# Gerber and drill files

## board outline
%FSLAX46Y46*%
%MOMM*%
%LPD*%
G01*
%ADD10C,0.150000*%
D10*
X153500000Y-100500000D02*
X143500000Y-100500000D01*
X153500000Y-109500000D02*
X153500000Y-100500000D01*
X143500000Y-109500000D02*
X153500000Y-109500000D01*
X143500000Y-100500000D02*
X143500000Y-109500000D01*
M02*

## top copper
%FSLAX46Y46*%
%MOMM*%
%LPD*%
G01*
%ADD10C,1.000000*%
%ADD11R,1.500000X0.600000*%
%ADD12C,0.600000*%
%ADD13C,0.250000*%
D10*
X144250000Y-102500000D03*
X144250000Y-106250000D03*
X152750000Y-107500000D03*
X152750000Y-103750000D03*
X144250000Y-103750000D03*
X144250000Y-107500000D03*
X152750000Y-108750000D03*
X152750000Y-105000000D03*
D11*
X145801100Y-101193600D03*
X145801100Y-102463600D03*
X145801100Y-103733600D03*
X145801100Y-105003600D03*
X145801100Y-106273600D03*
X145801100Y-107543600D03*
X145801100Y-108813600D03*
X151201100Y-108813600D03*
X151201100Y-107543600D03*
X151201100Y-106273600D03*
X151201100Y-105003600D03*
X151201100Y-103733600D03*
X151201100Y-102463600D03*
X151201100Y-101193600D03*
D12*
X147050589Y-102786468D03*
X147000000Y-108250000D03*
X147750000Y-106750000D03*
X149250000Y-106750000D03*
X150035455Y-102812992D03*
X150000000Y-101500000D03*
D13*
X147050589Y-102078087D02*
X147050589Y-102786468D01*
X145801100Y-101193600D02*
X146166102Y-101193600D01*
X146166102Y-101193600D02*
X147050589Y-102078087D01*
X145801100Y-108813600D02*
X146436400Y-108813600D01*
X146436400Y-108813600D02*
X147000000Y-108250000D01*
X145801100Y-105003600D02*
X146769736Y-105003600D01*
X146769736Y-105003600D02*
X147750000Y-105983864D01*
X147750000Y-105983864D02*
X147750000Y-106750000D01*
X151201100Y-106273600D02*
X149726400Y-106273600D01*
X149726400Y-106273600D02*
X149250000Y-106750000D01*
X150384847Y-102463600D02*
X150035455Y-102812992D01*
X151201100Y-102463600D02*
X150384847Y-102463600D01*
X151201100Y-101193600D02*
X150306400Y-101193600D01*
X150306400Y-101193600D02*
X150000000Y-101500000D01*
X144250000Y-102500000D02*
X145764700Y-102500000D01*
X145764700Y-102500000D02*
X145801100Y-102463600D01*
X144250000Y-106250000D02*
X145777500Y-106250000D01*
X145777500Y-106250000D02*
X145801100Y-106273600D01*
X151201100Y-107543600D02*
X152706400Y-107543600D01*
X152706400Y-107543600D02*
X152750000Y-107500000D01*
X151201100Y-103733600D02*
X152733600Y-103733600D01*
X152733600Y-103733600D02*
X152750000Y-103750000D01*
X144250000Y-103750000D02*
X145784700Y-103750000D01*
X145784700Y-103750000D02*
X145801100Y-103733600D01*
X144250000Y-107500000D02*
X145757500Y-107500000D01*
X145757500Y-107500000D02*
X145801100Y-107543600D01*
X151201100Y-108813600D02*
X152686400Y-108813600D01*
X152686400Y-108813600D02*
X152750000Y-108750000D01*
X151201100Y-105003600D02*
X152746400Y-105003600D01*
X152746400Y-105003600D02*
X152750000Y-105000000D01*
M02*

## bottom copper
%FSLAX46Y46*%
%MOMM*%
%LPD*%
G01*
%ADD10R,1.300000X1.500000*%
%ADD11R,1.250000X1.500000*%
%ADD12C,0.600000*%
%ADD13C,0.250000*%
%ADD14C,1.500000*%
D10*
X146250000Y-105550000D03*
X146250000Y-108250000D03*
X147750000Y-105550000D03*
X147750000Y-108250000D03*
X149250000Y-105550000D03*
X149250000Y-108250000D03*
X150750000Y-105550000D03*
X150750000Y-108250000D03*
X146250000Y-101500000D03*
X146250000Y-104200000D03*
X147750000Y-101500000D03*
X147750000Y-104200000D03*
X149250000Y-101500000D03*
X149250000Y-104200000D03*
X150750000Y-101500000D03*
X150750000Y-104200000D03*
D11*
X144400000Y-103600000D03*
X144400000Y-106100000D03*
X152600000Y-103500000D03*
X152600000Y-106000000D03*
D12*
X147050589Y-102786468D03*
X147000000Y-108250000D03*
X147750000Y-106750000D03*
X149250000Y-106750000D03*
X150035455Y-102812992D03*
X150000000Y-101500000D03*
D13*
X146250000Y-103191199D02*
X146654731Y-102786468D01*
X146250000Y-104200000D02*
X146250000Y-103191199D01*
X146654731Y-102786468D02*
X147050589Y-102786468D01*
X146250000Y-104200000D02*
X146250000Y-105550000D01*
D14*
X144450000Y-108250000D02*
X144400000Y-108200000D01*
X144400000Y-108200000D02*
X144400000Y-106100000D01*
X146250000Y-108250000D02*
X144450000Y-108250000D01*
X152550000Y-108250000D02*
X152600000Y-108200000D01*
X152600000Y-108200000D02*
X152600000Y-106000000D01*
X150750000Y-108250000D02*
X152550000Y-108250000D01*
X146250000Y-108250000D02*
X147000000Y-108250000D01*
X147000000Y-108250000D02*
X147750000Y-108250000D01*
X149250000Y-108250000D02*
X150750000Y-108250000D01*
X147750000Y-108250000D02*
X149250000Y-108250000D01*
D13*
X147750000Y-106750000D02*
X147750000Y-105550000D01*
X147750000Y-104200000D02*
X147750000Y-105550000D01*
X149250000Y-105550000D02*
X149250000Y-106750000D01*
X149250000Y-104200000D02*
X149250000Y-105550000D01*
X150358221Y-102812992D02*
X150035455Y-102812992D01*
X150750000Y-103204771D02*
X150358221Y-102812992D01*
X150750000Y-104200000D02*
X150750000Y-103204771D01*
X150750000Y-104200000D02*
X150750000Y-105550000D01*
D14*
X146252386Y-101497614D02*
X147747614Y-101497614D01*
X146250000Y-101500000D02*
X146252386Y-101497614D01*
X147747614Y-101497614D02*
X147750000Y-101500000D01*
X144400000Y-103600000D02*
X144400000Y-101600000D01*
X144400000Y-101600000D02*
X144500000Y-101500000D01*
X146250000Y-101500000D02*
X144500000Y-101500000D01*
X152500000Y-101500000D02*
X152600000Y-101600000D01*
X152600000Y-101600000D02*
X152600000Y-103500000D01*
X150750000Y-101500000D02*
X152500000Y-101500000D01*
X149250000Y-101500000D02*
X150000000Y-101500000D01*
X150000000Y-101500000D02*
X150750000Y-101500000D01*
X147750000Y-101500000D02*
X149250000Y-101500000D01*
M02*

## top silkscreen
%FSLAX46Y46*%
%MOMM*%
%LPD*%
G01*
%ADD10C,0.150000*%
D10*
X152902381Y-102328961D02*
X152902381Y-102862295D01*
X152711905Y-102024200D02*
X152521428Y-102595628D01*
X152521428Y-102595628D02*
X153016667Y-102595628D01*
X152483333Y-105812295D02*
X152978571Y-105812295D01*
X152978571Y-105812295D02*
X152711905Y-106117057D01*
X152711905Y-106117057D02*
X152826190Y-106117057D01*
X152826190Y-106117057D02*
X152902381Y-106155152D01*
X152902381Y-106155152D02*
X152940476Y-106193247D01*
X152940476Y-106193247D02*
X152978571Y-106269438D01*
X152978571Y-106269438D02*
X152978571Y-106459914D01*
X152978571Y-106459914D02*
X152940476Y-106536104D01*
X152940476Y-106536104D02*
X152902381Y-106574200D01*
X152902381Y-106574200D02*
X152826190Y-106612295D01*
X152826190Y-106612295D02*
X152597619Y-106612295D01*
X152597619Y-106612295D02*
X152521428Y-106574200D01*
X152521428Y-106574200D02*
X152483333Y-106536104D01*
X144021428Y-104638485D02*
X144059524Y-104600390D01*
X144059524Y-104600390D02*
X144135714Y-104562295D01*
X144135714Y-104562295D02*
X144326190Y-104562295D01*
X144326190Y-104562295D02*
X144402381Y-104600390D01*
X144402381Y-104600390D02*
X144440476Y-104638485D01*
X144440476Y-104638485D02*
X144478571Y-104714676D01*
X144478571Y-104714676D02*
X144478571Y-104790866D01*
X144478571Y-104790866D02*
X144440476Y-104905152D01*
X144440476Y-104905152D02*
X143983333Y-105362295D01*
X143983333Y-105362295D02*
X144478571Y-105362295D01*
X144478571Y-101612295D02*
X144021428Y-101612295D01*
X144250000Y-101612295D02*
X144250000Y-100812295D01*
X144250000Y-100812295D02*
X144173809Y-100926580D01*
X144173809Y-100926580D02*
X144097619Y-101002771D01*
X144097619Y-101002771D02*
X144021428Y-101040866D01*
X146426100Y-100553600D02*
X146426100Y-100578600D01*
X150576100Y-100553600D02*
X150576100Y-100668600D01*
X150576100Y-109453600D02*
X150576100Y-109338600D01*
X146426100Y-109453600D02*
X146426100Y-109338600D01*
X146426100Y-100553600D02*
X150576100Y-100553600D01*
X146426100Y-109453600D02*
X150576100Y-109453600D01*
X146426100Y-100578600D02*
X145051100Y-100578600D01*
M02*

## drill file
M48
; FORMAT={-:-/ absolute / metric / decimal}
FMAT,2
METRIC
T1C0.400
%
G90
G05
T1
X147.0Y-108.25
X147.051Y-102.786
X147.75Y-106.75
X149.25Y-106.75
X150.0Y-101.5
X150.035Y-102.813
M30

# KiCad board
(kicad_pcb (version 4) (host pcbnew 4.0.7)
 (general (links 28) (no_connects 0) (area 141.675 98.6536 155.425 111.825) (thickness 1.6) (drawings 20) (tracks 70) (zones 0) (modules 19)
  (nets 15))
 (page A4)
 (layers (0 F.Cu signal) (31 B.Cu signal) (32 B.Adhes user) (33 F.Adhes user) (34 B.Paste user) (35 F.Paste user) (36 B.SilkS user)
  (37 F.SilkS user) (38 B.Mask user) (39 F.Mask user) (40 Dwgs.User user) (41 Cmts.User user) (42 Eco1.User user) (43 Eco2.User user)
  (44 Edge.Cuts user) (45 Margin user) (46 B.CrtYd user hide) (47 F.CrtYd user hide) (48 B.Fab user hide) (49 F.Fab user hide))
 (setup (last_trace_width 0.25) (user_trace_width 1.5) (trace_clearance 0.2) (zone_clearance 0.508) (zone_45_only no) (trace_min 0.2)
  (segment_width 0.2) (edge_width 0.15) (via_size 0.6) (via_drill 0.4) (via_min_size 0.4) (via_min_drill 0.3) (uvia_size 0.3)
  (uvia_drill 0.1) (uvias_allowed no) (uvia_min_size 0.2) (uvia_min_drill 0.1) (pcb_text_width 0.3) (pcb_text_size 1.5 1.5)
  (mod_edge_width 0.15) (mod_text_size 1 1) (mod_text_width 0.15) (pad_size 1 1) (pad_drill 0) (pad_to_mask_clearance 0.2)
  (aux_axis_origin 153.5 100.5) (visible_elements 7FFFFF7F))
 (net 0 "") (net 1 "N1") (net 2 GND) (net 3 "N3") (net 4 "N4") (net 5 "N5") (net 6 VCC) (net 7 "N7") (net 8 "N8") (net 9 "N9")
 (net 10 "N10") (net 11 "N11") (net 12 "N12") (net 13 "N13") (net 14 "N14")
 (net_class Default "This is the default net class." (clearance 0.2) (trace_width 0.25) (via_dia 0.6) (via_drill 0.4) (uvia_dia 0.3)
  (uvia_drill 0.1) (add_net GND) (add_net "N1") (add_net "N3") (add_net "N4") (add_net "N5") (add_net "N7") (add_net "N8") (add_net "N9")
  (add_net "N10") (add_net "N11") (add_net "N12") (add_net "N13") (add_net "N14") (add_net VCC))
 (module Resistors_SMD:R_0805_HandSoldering (layer B.Cu) (at 146.25 106.9 270)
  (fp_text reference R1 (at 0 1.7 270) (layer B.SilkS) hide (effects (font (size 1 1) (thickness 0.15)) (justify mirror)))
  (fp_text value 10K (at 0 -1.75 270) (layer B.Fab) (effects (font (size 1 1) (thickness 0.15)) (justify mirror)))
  (pad 1 smd rect (at -1.35 0 270) (size 1.5 1.3) (layers B.Cu B.Paste B.Mask) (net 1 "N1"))
  (pad 2 smd rect (at 1.35 0 270) (size 1.5 1.3) (layers B.Cu B.Paste B.Mask) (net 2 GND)))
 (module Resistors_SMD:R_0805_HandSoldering (layer B.Cu) (at 147.75 106.9 270)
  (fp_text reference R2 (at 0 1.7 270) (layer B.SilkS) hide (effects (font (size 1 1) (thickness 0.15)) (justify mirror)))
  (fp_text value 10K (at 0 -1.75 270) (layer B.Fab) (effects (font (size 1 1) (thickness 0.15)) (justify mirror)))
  (pad 1 smd rect (at -1.35 0 270) (size 1.5 1.3) (layers B.Cu B.Paste B.Mask) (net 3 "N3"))
  (pad 2 smd rect (at 1.35 0 270) (size 1.5 1.3) (layers B.Cu B.Paste B.Mask) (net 2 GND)))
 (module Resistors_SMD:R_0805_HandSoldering (layer B.Cu) (at 149.25 106.9 270)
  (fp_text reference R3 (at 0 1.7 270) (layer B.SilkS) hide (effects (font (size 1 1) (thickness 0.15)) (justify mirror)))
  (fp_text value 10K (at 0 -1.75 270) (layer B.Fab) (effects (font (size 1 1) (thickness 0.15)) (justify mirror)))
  (pad 1 smd rect (at -1.35 0 270) (size 1.5 1.3) (layers B.Cu B.Paste B.Mask) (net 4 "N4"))
  (pad 2 smd rect (at 1.35 0 270) (size 1.5 1.3) (layers B.Cu B.Paste B.Mask) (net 2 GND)))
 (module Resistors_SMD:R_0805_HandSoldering (layer B.Cu) (at 150.75 106.9 270)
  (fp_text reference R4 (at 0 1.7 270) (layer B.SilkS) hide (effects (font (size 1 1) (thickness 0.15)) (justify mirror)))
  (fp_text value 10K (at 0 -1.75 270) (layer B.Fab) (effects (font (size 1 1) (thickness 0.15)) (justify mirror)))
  (pad 1 smd rect (at -1.35 0 270) (size 1.5 1.3) (layers B.Cu B.Paste B.Mask) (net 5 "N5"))
  (pad 2 smd rect (at 1.35 0 270) (size 1.5 1.3) (layers B.Cu B.Paste B.Mask) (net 2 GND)))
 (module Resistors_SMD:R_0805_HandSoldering (layer B.Cu) (at 146.25 102.85 270)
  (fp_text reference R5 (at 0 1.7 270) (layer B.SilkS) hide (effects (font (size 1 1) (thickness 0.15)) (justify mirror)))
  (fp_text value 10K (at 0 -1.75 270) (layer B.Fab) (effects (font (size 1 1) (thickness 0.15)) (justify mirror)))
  (pad 1 smd rect (at -1.35 0 270) (size 1.5 1.3) (layers B.Cu B.Paste B.Mask) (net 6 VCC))
  (pad 2 smd rect (at 1.35 0 270) (size 1.5 1.3) (layers B.Cu B.Paste B.Mask) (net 1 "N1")))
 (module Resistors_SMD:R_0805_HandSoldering (layer B.Cu) (at 147.75 102.85 270)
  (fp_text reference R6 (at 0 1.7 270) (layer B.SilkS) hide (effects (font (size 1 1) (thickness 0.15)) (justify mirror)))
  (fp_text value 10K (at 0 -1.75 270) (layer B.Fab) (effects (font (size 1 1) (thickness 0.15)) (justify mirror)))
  (pad 1 smd rect (at -1.35 0 270) (size 1.5 1.3) (layers B.Cu B.Paste B.Mask) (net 6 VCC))
  (pad 2 smd rect (at 1.35 0 270) (size 1.5 1.3) (layers B.Cu B.Paste B.Mask) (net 3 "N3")))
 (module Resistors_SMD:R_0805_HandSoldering (layer B.Cu) (at 149.25 102.85 270)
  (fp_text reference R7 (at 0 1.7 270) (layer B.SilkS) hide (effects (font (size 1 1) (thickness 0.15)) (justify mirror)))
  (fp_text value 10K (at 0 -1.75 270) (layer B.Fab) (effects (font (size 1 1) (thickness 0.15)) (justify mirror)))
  (pad 1 smd rect (at -1.35 0 270) (size 1.5 1.3) (layers B.Cu B.Paste B.Mask) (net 6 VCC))
  (pad 2 smd rect (at 1.35 0 270) (size 1.5 1.3) (layers B.Cu B.Paste B.Mask) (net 4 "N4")))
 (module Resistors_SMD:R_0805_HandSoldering (layer B.Cu) (at 150.75 102.85 270)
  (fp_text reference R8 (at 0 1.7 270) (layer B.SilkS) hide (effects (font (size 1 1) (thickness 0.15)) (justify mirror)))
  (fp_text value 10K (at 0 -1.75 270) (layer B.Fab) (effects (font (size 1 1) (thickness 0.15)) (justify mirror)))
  (pad 1 smd rect (at -1.35 0 270) (size 1.5 1.3) (layers B.Cu B.Paste B.Mask) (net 6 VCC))
  (pad 2 smd rect (at 1.35 0 270) (size 1.5 1.3) (layers B.Cu B.Paste B.Mask) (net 5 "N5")))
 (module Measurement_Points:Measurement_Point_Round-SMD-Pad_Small (layer F.Cu) (at 144.25 102.5)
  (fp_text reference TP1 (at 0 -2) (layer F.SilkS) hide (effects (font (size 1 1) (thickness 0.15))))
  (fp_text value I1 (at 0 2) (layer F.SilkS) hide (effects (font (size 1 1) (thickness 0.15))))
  (pad 1 smd circle (at 0 0) (size 1 1) (layers F.Cu F.Mask) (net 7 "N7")))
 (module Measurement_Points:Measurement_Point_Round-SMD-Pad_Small (layer F.Cu) (at 144.25 106.25)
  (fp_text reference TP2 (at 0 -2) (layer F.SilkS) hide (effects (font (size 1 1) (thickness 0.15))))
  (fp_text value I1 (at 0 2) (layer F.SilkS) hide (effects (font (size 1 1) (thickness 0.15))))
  (pad 1 smd circle (at 0 0) (size 1 1) (layers F.Cu F.Mask) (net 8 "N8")))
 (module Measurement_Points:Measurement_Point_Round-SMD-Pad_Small (layer F.Cu) (at 152.75 107.5)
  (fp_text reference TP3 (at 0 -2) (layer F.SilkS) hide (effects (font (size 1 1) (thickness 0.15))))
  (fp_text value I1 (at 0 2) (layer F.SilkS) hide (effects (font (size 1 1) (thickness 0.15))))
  (pad 1 smd circle (at 0 0) (size 1 1) (layers F.Cu F.Mask) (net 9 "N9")))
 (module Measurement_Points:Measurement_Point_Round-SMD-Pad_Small (layer F.Cu) (at 152.75 103.75)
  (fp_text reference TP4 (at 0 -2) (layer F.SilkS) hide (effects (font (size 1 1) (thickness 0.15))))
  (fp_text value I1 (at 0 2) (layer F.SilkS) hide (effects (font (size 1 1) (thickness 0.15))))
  (pad 1 smd circle (at 0 0) (size 1 1) (layers F.Cu F.Mask) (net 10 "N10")))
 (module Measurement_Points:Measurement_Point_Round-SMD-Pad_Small (layer F.Cu) (at 144.25 103.75)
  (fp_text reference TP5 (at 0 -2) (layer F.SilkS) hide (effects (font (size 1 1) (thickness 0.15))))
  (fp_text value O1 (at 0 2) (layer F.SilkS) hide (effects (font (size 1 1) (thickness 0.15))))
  (pad 1 smd circle (at 0 0) (size 1 1) (layers F.Cu F.Mask) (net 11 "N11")))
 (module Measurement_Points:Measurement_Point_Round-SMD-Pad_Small (layer F.Cu) (at 144.25 107.5)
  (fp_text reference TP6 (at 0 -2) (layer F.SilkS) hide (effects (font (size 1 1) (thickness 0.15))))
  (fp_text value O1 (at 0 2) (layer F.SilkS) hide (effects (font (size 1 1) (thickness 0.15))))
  (pad 1 smd circle (at 0 0) (size 1 1) (layers F.Cu F.Mask) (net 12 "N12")))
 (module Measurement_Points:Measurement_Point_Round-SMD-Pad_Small (layer F.Cu) (at 152.75 108.75)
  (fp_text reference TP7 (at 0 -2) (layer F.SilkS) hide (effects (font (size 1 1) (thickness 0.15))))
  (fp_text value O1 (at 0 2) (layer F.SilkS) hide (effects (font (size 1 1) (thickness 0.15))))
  (pad 1 smd circle (at 0 0) (size 1 1) (layers F.Cu F.Mask) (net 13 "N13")))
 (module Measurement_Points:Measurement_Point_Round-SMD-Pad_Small (layer F.Cu) (at 152.75 105)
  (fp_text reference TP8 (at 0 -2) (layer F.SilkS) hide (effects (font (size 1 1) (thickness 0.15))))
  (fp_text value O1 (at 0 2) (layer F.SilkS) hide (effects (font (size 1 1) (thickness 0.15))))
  (pad 1 smd circle (at 0 0) (size 1 1) (layers F.Cu F.Mask) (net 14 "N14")))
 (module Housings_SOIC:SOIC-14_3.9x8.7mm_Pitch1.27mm (layer F.Cu) (at 148.5011 105.0036)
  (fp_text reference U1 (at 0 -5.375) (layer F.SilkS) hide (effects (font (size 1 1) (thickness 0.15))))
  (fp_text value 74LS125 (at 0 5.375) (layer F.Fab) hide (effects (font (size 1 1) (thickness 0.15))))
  (fp_line (start -2.075 -4.45) (end -2.075 -4.425) (layer F.SilkS) (width 0.15))
  (fp_line (start 2.075 -4.45) (end 2.075 -4.335) (layer F.SilkS) (width 0.15))
  (fp_line (start 2.075 4.45) (end 2.075 4.335) (layer F.SilkS) (width 0.15))
  (fp_line (start -2.075 4.45) (end -2.075 4.335) (layer F.SilkS) (width 0.15))
  (fp_line (start -2.075 -4.45) (end 2.075 -4.45) (layer F.SilkS) (width 0.15))
  (fp_line (start -2.075 4.45) (end 2.075 4.45) (layer F.SilkS) (width 0.15))
  (fp_line (start -2.075 -4.425) (end -3.45 -4.425) (layer F.SilkS) (width 0.15))
  (pad 1 smd rect (at -2.7 -3.81) (size 1.5 0.6) (layers F.Cu F.Paste F.Mask) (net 1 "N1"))
  (pad 2 smd rect (at -2.7 -2.54) (size 1.5 0.6) (layers F.Cu F.Paste F.Mask) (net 7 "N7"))
  (pad 3 smd rect (at -2.7 -1.27) (size 1.5 0.6) (layers F.Cu F.Paste F.Mask) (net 11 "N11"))
  (pad 4 smd rect (at -2.7 0) (size 1.5 0.6) (layers F.Cu F.Paste F.Mask) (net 3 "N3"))
  (pad 5 smd rect (at -2.7 1.27) (size 1.5 0.6) (layers F.Cu F.Paste F.Mask) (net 8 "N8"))
  (pad 6 smd rect (at -2.7 2.54) (size 1.5 0.6) (layers F.Cu F.Paste F.Mask) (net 12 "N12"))
  (pad 7 smd rect (at -2.7 3.81) (size 1.5 0.6) (layers F.Cu F.Paste F.Mask) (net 2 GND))
  (pad 8 smd rect (at 2.7 3.81) (size 1.5 0.6) (layers F.Cu F.Paste F.Mask) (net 13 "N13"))
  (pad 9 smd rect (at 2.7 2.54) (size 1.5 0.6) (layers F.Cu F.Paste F.Mask) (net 9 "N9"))
  (pad 10 smd rect (at 2.7 1.27) (size 1.5 0.6) (layers F.Cu F.Paste F.Mask) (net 4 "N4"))
  (pad 11 smd rect (at 2.7 0) (size 1.5 0.6) (layers F.Cu F.Paste F.Mask) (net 14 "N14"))
  (pad 12 smd rect (at 2.7 -1.27) (size 1.5 0.6) (layers F.Cu F.Paste F.Mask) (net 10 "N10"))
  (pad 13 smd rect (at 2.7 -2.54) (size 1.5 0.6) (layers F.Cu F.Paste F.Mask) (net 5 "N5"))
  (pad 14 smd rect (at 2.7 -3.81) (size 1.5 0.6) (layers F.Cu F.Paste F.Mask) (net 6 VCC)))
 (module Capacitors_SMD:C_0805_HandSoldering (layer B.Cu) (at 144.4 104.85 270)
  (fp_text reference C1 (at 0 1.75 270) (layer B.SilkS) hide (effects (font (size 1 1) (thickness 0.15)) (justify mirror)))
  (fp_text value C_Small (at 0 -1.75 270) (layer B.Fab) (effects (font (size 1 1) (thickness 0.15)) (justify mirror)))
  (pad 1 smd rect (at -1.25 0 270) (size 1.5 1.25) (layers B.Cu B.Paste B.Mask) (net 6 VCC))
  (pad 2 smd rect (at 1.25 0 270) (size 1.5 1.25) (layers B.Cu B.Paste B.Mask) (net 2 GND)))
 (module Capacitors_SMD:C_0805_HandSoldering (layer B.Cu) (at 152.6 104.75 270)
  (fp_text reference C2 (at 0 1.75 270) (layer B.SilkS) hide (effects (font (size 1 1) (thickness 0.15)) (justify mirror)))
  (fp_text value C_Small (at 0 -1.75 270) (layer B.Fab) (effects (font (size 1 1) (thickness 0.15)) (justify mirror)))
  (pad 1 smd rect (at -1.25 0 270) (size 1.5 1.25) (layers B.Cu B.Paste B.Mask) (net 6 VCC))
  (pad 2 smd rect (at 1.25 0 270) (size 1.5 1.25) (layers B.Cu B.Paste B.Mask) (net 2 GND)))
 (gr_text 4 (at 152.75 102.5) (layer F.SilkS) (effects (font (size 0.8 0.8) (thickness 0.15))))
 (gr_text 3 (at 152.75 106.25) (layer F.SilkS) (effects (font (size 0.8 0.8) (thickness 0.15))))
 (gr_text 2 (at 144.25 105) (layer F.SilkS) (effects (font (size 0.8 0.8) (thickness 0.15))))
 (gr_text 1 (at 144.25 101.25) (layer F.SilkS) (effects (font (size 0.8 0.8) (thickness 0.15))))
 (gr_line (start 153.5 100.5) (end 143.5 100.5) (layer Edge.Cuts) (width 0.15))
 (gr_line (start 153.5 109.5) (end 153.5 100.5) (layer Edge.Cuts) (width 0.15))
 (gr_line (start 143.5 109.5) (end 153.5 109.5) (layer Edge.Cuts) (width 0.15))
 (gr_line (start 143.5 100.5) (end 143.5 109.5) (layer Edge.Cuts) (width 0.15))
 (segment (start 146.25 103.191199) (end 146.654731 102.786468) (width 0.25) (layer B.Cu) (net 1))
 (segment (start 147.050589 102.078087) (end 147.050589 102.786468) (width 0.25) (layer F.Cu) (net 1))
 (segment (start 146.25 104.2) (end 146.25 103.191199) (width 0.25) (layer B.Cu) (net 1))
 (via (at 147.050589 102.786468) (size 0.6) (drill 0.4) (layers F.Cu B.Cu) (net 1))
 (segment (start 146.654731 102.786468) (end 147.050589 102.786468) (width 0.25) (layer B.Cu) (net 1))
 (segment (start 145.8011 101.1936) (end 146.166102 101.1936) (width 0.25) (layer F.Cu) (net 1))
 (segment (start 146.166102 101.1936) (end 147.050589 102.078087) (width 0.25) (layer F.Cu) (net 1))
 (segment (start 146.25 104.2) (end 146.25 105.55) (width 0.25) (layer B.Cu) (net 1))
 (segment (start 144.45 108.25) (end 144.4 108.2) (width 1.5) (layer B.Cu) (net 2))
 (segment (start 144.4 108.2) (end 144.4 106.1) (width 1.5) (layer B.Cu) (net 2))
 (segment (start 146.25 108.25) (end 144.45 108.25) (width 1.5) (layer B.Cu) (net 2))
 (segment (start 152.55 108.25) (end 152.6 108.2) (width 1.5) (layer B.Cu) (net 2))
 (segment (start 152.6 108.2) (end 152.6 106) (width 1.5) (layer B.Cu) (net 2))
 (segment (start 150.75 108.25) (end 152.55 108.25) (width 1.5) (layer B.Cu) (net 2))
 (segment (start 146.25 108.25) (end 147 108.25) (width 1.5) (layer B.Cu) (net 2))
 (segment (start 147 108.25) (end 147.75 108.25) (width 1.5) (layer B.Cu) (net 2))
 (segment (start 145.8011 108.8136) (end 146.4364 108.8136) (width 0.25) (layer F.Cu) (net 2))
 (segment (start 146.4364 108.8136) (end 147 108.25) (width 0.25) (layer F.Cu) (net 2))
 (via (at 147 108.25) (size 0.6) (drill 0.4) (layers F.Cu B.Cu) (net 2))
 (segment (start 149.25 108.25) (end 150.75 108.25) (width 1.5) (layer B.Cu) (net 2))
 (segment (start 147.75 108.25) (end 149.25 108.25) (width 1.5) (layer B.Cu) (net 2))
 (segment (start 145.8011 105.0036) (end 146.769736 105.0036) (width 0.25) (layer F.Cu) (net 3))
 (segment (start 146.769736 105.0036) (end 147.75 105.983864) (width 0.25) (layer F.Cu) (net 3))
 (segment (start 147.75 105.983864) (end 147.75 106.75) (width 0.25) (layer F.Cu) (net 3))
 (segment (start 147.75 106.75) (end 147.75 105.55) (width 0.25) (layer B.Cu) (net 3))
 (via (at 147.75 106.75) (size 0.6) (drill 0.4) (layers F.Cu B.Cu) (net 3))
 (segment (start 147.75 104.2) (end 147.75 105.55) (width 0.25) (layer B.Cu) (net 3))
 (segment (start 151.2011 106.2736) (end 149.7264 106.2736) (width 0.25) (layer F.Cu) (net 4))
 (segment (start 149.7264 106.2736) (end 149.25 106.75) (width 0.25) (layer F.Cu) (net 4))
 (segment (start 149.25 105.55) (end 149.25 106.75) (width 0.25) (layer B.Cu) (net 4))
 (via (at 149.25 106.75) (size 0.6) (drill 0.4) (layers F.Cu B.Cu) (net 4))
 (segment (start 149.25 104.2) (end 149.25 105.55) (width 0.25) (layer B.Cu) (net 4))
 (segment (start 150.358221 102.812992) (end 150.035455 102.812992) (width 0.25) (layer B.Cu) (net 5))
 (segment (start 150.75 103.204771) (end 150.358221 102.812992) (width 0.25) (layer B.Cu) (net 5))
 (segment (start 150.75 104.2) (end 150.75 103.204771) (width 0.25) (layer B.Cu) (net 5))
 (segment (start 150.384847 102.4636) (end 150.035455 102.812992) (width 0.25) (layer F.Cu) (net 5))
 (via (at 150.035455 102.812992) (size 0.6) (drill 0.4) (layers F.Cu B.Cu) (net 5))
 (segment (start 151.2011 102.4636) (end 150.384847 102.4636) (width 0.25) (layer F.Cu) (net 5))
 (segment (start 150.75 104.2) (end 150.75 105.55) (width 0.25) (layer B.Cu) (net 5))
 (segment (start 146.252386 101.497614) (end 147.747614 101.497614) (width 1.5) (layer B.Cu) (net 6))
 (segment (start 146.25 101.5) (end 146.252386 101.497614) (width 1.5) (layer B.Cu) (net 6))
 (segment (start 147.747614 101.497614) (end 147.75 101.5) (width 1.5) (layer B.Cu) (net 6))
 (segment (start 144.4 103.6) (end 144.4 101.6) (width 1.5) (layer B.Cu) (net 6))
 (segment (start 144.4 101.6) (end 144.5 101.5) (width 1.5) (layer B.Cu) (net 6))
 (segment (start 146.25 101.5) (end 144.5 101.5) (width 1.5) (layer B.Cu) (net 6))
 (segment (start 152.5 101.5) (end 152.6 101.6) (width 1.5) (layer B.Cu) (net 6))
 (segment (start 152.6 101.6) (end 152.6 103.5) (width 1.5) (layer B.Cu) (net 6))
 (segment (start 150.75 101.5) (end 152.5 101.5) (width 1.5) (layer B.Cu) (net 6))
 (segment (start 149.25 101.5) (end 150 101.5) (width 1.5) (layer B.Cu) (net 6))
 (segment (start 150 101.5) (end 150.75 101.5) (width 1.5) (layer B.Cu) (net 6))
 (segment (start 151.2011 101.1936) (end 150.3064 101.1936) (width 0.25) (layer F.Cu) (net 6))
 (segment (start 150.3064 101.1936) (end 150 101.5) (width 0.25) (layer F.Cu) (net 6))
 (via (at 150 101.5) (size 0.6) (drill 0.4) (layers F.Cu B.Cu) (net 6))
 (segment (start 147.75 101.5) (end 149.25 101.5) (width 1.5) (layer B.Cu) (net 6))
 (segment (start 144.25 102.5) (end 145.7647 102.5) (width 0.25) (layer F.Cu) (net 7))
 (segment (start 145.7647 102.5) (end 145.8011 102.4636) (width 0.25) (layer F.Cu) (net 7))
 (segment (start 144.25 106.25) (end 145.7775 106.25) (width 0.25) (layer F.Cu) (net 8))
 (segment (start 145.7775 106.25) (end 145.8011 106.2736) (width 0.25) (layer F.Cu) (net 8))
 (segment (start 151.2011 107.5436) (end 152.7064 107.5436) (width 0.25) (layer F.Cu) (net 9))
 (segment (start 152.7064 107.5436) (end 152.75 107.5) (width 0.25) (layer F.Cu) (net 9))
 (segment (start 151.2011 103.7336) (end 152.7336 103.7336) (width 0.25) (layer F.Cu) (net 10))
 (segment (start 152.7336 103.7336) (end 152.75 103.75) (width 0.25) (layer F.Cu) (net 10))
 (segment (start 144.25 103.75) (end 145.7847 103.75) (width 0.25) (layer F.Cu) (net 11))
 (segment (start 145.7847 103.75) (end 145.8011 103.7336) (width 0.25) (layer F.Cu) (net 11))
 (segment (start 144.25 107.5) (end 145.7575 107.5) (width 0.25) (layer F.Cu) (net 12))
 (segment (start 145.7575 107.5) (end 145.8011 107.5436) (width 0.25) (layer F.Cu) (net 12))
 (segment (start 151.2011 108.8136) (end 152.6864 108.8136) (width 0.25) (layer F.Cu) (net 13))
 (segment (start 152.6864 108.8136) (end 152.75 108.75) (width 0.25) (layer F.Cu) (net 13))
 (segment (start 151.2011 105.0036) (end 152.7464 105.0036) (width 0.25) (layer F.Cu) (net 14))
 (segment (start 152.7464 105.0036) (end 152.75 105) (width 0.25) (layer F.Cu) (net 14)))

